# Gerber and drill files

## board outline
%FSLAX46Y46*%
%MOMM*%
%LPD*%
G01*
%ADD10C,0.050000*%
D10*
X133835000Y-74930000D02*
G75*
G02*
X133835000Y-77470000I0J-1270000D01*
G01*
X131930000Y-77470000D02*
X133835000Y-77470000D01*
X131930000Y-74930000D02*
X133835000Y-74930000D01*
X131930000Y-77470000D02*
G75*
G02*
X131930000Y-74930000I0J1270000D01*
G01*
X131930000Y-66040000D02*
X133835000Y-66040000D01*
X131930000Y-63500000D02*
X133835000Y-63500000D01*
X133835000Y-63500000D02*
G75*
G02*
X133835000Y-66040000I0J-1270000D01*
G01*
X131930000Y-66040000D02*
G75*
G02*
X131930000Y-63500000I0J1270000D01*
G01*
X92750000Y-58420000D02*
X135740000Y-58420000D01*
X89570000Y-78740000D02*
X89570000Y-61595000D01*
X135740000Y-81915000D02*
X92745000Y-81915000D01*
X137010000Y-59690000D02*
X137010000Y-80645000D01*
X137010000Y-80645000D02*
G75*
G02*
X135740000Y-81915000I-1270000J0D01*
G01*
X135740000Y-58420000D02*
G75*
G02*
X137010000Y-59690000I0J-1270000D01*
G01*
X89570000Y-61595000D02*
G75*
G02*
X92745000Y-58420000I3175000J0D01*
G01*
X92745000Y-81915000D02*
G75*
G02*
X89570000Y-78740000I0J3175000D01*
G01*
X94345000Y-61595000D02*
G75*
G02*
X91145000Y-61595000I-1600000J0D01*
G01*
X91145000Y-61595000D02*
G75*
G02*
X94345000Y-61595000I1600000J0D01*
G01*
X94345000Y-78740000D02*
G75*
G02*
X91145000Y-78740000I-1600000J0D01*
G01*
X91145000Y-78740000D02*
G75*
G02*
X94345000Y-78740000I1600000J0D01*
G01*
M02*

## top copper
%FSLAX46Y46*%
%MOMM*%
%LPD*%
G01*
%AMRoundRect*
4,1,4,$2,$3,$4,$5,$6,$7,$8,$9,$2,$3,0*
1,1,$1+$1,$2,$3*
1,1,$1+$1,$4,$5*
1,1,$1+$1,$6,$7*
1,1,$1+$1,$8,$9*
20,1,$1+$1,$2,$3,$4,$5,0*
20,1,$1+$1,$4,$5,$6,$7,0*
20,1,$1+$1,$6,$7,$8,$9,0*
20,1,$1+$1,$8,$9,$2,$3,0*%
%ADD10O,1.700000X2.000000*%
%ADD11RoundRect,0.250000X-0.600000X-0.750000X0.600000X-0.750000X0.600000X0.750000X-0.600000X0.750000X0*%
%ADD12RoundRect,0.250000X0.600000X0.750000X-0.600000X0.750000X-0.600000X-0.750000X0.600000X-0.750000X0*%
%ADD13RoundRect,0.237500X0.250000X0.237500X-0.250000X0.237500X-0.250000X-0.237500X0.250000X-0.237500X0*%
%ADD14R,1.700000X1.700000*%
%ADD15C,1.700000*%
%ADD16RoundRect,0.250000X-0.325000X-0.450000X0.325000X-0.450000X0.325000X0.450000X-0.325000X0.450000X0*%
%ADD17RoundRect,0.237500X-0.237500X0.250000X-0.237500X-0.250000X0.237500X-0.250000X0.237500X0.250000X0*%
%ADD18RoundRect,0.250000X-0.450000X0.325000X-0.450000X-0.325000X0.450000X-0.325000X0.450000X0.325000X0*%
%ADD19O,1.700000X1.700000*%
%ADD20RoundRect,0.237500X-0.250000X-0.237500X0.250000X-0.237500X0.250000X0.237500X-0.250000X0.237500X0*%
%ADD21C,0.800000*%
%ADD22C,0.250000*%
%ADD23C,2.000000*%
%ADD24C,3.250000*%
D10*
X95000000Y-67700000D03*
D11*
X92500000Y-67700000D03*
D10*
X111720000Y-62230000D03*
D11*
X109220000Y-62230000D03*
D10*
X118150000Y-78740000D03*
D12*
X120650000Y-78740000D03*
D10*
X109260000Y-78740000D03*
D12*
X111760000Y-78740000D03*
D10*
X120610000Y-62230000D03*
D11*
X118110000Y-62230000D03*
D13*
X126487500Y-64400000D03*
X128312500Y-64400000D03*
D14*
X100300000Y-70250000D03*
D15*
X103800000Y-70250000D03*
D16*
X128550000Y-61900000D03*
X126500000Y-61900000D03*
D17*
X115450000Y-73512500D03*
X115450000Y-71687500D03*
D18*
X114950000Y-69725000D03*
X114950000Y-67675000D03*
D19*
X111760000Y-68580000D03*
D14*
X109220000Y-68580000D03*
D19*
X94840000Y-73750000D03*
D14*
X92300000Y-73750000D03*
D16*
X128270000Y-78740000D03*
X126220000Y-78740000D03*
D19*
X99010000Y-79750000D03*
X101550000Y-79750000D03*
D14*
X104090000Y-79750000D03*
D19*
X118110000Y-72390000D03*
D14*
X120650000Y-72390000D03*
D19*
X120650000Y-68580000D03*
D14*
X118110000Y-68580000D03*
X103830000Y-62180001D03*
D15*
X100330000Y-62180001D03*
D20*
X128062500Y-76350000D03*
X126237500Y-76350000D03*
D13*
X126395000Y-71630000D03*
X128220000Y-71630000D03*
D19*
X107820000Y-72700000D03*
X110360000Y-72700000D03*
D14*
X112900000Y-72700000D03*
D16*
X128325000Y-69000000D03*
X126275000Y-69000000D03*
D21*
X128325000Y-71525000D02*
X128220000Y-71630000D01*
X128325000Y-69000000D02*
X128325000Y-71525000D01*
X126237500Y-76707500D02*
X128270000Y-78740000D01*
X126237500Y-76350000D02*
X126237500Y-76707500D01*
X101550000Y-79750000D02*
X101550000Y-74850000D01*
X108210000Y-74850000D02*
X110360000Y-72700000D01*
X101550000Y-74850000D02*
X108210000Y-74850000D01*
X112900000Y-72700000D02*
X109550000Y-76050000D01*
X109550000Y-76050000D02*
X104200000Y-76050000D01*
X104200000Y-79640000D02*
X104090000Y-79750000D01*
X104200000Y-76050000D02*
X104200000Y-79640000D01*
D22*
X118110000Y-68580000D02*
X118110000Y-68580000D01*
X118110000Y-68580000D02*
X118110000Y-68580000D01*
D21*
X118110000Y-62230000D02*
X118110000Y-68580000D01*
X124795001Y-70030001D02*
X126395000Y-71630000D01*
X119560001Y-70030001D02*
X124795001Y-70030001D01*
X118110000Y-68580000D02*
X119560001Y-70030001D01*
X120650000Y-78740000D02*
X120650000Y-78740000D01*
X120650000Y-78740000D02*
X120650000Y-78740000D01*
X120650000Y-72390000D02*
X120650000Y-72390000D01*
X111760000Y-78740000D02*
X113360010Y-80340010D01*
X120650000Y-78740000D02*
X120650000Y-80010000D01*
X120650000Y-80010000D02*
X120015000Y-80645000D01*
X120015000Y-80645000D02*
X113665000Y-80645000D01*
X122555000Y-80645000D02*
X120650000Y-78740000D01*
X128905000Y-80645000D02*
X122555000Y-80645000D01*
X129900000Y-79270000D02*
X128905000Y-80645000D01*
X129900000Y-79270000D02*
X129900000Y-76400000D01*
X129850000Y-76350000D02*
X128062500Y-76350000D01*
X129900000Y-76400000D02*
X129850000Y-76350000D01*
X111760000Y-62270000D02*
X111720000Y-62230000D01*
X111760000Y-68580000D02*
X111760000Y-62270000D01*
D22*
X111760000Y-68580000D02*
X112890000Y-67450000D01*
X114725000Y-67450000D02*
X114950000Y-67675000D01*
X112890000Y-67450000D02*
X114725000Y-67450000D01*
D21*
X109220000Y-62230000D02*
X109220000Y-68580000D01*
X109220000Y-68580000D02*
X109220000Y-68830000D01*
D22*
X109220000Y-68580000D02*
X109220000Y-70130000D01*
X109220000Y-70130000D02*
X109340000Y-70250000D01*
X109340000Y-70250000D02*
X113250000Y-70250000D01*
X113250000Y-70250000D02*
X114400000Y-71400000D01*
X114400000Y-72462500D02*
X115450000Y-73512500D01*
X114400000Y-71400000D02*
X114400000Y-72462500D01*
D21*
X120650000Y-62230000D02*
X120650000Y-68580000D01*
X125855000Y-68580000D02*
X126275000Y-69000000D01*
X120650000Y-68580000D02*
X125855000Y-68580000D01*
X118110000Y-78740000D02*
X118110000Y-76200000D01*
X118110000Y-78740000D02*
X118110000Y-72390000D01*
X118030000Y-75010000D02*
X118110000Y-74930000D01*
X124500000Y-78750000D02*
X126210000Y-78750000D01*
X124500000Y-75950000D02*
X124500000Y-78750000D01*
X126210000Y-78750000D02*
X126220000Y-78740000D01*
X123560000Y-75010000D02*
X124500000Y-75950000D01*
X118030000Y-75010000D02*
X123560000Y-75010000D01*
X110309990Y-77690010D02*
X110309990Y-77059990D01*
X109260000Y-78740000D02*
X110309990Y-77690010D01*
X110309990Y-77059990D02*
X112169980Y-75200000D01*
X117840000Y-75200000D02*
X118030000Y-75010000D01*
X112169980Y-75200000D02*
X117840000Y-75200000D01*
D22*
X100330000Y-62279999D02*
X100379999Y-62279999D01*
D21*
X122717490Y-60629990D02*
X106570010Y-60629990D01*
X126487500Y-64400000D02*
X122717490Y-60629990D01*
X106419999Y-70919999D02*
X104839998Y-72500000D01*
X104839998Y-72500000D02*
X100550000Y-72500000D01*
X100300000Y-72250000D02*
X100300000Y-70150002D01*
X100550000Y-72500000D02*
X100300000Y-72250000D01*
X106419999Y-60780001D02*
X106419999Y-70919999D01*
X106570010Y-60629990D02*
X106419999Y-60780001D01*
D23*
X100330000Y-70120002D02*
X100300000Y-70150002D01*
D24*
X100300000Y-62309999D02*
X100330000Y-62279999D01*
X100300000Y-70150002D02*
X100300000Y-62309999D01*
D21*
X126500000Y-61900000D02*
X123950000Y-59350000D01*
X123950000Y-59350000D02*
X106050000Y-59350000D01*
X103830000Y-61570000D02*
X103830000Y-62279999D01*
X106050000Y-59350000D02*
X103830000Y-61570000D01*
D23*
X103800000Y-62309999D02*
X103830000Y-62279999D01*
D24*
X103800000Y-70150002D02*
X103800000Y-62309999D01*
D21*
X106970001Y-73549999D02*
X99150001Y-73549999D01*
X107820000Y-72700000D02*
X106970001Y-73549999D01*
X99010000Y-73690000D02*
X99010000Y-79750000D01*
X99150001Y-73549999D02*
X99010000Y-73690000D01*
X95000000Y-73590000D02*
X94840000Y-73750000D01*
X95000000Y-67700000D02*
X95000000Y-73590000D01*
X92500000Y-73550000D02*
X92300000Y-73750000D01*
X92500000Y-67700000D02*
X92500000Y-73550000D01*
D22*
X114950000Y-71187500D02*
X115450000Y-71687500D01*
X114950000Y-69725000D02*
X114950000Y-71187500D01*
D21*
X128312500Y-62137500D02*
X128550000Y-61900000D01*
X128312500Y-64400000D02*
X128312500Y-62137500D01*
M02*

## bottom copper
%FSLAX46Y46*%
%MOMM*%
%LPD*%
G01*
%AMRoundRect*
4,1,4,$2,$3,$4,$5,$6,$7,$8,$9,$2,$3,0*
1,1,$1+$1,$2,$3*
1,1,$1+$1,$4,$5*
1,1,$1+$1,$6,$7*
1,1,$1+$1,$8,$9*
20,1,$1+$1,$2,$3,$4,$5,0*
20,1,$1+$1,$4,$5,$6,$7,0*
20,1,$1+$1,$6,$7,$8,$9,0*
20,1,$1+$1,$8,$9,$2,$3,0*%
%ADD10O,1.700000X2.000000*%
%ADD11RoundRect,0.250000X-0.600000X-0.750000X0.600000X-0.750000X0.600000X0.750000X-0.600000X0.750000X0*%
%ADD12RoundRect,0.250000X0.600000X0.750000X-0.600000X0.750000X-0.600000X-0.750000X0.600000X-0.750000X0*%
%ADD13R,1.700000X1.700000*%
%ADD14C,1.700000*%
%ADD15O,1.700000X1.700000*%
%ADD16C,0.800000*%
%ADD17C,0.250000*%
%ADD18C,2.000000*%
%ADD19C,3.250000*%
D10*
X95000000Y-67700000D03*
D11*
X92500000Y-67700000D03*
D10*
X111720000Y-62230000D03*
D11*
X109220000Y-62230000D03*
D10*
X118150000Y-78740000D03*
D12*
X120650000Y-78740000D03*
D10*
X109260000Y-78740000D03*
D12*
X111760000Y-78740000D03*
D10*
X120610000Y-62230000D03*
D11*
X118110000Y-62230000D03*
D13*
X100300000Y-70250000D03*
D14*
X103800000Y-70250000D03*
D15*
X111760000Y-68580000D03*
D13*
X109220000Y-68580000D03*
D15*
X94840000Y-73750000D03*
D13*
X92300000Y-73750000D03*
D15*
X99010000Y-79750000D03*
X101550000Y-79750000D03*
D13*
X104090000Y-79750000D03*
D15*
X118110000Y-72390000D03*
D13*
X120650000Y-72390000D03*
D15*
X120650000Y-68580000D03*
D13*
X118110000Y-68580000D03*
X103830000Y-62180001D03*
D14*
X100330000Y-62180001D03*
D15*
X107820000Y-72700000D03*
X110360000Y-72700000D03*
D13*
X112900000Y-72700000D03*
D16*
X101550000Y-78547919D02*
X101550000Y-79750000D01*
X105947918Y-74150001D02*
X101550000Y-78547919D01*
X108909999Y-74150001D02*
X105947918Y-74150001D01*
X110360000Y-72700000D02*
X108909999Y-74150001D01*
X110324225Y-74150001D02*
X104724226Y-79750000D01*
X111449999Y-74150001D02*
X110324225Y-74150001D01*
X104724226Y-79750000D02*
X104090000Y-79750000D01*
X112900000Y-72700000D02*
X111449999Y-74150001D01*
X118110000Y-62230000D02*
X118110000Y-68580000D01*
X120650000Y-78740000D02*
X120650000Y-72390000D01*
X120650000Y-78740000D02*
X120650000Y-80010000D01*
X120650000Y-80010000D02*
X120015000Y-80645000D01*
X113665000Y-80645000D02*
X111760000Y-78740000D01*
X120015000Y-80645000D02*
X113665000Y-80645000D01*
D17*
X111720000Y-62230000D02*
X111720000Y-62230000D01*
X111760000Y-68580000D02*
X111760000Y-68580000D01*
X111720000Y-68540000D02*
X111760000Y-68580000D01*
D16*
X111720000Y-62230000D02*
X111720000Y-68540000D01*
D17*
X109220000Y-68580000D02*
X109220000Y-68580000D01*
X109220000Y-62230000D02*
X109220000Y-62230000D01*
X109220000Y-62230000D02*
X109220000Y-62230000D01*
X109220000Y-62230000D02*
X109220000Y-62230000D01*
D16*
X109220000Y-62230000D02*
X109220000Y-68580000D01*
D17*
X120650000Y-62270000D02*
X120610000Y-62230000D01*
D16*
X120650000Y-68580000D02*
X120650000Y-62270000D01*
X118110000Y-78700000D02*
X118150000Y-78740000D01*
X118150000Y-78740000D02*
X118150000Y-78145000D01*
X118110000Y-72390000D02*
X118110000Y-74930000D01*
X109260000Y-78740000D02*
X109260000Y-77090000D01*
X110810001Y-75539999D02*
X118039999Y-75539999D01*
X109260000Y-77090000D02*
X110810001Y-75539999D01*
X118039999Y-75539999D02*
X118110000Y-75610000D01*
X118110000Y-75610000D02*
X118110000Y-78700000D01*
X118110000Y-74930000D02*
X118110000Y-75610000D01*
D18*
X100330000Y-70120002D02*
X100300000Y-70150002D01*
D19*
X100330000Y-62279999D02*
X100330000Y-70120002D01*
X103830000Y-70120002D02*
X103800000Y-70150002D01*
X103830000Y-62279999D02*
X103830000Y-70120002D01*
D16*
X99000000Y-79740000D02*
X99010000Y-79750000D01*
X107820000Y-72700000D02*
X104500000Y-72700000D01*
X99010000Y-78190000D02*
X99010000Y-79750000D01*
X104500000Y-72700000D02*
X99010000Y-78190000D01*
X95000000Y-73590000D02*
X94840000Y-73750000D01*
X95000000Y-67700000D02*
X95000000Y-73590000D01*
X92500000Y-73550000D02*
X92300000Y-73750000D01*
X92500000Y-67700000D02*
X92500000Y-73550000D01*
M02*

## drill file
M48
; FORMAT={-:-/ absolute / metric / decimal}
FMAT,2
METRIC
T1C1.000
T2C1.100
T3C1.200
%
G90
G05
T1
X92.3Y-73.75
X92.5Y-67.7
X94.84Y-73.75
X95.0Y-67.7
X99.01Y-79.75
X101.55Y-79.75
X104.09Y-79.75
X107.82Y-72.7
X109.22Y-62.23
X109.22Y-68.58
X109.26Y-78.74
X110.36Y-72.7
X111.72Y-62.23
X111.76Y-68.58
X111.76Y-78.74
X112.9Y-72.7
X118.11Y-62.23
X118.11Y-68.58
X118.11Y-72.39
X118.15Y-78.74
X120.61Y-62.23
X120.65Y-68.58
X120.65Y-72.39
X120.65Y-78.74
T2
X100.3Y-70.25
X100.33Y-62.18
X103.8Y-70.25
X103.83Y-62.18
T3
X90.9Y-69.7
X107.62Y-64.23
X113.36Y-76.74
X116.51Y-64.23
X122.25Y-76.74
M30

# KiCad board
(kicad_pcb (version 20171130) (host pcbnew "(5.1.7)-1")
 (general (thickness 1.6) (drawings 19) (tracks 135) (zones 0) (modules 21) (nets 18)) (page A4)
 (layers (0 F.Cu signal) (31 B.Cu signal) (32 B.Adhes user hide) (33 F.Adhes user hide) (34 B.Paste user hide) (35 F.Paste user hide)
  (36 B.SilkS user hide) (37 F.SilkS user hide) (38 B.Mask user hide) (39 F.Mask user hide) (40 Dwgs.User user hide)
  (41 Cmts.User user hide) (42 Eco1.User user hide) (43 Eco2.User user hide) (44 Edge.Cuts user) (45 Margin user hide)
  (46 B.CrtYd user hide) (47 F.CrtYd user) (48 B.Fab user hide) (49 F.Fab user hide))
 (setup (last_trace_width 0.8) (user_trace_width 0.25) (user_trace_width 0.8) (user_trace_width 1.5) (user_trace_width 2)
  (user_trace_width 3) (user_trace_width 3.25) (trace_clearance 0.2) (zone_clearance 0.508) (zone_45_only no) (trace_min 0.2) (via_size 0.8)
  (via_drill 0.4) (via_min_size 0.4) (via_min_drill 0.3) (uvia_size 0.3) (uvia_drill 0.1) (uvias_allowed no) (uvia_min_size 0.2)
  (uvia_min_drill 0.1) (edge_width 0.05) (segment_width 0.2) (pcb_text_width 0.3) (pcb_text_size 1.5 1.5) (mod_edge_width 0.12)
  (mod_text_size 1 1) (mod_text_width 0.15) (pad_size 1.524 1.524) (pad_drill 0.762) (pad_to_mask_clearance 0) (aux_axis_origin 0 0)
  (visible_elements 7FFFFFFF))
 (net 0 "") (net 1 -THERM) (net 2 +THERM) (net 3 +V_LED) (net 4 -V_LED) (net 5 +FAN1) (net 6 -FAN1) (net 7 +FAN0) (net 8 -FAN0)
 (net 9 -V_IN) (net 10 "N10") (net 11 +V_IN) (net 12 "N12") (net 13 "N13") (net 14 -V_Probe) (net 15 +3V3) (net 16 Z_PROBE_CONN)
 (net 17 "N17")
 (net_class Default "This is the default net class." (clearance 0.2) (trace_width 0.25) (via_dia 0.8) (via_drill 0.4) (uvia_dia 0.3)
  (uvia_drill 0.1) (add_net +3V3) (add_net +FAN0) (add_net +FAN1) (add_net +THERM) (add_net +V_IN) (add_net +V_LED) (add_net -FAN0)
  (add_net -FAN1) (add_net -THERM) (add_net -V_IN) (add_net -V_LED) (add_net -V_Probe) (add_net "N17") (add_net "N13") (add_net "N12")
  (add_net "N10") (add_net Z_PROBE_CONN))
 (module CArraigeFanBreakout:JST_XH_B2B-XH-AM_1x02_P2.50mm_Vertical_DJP (layer F.Cu) (at 92.5 67.7)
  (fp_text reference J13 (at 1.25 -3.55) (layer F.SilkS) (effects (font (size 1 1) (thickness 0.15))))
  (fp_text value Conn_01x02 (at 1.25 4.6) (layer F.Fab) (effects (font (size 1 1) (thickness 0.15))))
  (pad "" np_thru_hole circle (at -1.6 2) (size 1.2 1.2) (drill 1.2) (layers *.Cu *.Mask))
  (pad 2 thru_hole oval (at 2.5 0) (size 1.7 2) (drill 1) (layers *.Cu *.Mask) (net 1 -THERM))
  (pad 1 thru_hole roundrect (at 0 0) (size 1.7 2) (drill 1) (layers *.Cu *.Mask) (roundrect_rratio 0.147059) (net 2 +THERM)))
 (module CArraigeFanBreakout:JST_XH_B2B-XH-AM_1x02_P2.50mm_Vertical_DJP (layer F.Cu) (at 109.22 62.23)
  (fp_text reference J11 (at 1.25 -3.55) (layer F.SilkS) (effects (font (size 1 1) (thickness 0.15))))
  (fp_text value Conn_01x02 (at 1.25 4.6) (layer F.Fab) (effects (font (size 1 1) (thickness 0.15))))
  (pad "" np_thru_hole circle (at -1.6 2) (size 1.2 1.2) (drill 1.2) (layers *.Cu *.Mask))
  (pad 2 thru_hole oval (at 2.5 0) (size 1.7 2) (drill 1) (layers *.Cu *.Mask) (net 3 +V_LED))
  (pad 1 thru_hole roundrect (at 0 0) (size 1.7 2) (drill 1) (layers *.Cu *.Mask) (roundrect_rratio 0.147059) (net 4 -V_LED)))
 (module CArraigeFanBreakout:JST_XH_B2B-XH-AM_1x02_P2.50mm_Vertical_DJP (layer F.Cu) (at 120.65 78.74 180)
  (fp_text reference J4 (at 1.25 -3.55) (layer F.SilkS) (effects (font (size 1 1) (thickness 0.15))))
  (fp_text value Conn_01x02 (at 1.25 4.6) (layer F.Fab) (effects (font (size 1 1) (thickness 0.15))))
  (pad "" np_thru_hole circle (at -1.6 2 180) (size 1.2 1.2) (drill 1.2) (layers *.Cu *.Mask))
  (pad 2 thru_hole oval (at 2.5 0 180) (size 1.7 2) (drill 1) (layers *.Cu *.Mask) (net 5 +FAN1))
  (pad 1 thru_hole roundrect (at 0 0 180) (size 1.7 2) (drill 1) (layers *.Cu *.Mask) (roundrect_rratio 0.147059) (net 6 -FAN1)))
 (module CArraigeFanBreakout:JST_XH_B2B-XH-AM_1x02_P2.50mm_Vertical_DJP (layer F.Cu) (at 111.76 78.74 180)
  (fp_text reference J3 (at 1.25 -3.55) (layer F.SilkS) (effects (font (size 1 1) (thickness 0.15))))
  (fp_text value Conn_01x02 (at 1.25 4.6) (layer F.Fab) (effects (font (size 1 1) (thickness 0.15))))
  (pad "" np_thru_hole circle (at -1.6 2 180) (size 1.2 1.2) (drill 1.2) (layers *.Cu *.Mask))
  (pad 2 thru_hole oval (at 2.5 0 180) (size 1.7 2) (drill 1) (layers *.Cu *.Mask) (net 5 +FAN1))
  (pad 1 thru_hole roundrect (at 0 0 180) (size 1.7 2) (drill 1) (layers *.Cu *.Mask) (roundrect_rratio 0.147059) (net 6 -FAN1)))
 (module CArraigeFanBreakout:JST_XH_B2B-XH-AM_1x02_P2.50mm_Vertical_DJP (layer F.Cu) (at 118.11 62.23)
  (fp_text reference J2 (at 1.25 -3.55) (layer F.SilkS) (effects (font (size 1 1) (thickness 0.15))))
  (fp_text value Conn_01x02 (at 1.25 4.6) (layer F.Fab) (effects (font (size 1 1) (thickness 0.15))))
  (pad "" np_thru_hole circle (at -1.6 2) (size 1.2 1.2) (drill 1.2) (layers *.Cu *.Mask))
  (pad 2 thru_hole oval (at 2.5 0) (size 1.7 2) (drill 1) (layers *.Cu *.Mask) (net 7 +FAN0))
  (pad 1 thru_hole roundrect (at 0 0) (size 1.7 2) (drill 1) (layers *.Cu *.Mask) (roundrect_rratio 0.147059) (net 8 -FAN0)))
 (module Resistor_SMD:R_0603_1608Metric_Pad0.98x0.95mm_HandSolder (layer F.Cu) (at 127.4 64.4 180)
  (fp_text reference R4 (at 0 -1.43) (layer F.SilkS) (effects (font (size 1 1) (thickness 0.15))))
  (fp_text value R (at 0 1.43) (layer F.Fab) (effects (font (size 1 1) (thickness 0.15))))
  (pad 2 smd roundrect (at 0.9125 0 180) (size 0.975 0.95) (layers F.Cu F.Paste F.Mask) (roundrect_rratio 0.25) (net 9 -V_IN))
  (pad 1 smd roundrect (at -0.9125 0 180) (size 0.975 0.95) (layers F.Cu F.Paste F.Mask) (roundrect_rratio 0.25) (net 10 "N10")))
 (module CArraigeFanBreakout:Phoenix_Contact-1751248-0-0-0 (layer F.Cu) (at 102.05 70.200001)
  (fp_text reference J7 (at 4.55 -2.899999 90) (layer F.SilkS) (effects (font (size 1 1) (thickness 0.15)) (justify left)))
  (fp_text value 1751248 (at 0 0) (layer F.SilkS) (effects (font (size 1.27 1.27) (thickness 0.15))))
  (pad 1 thru_hole rect (at -1.75 0.049999) (size 1.7 1.7) (drill 1.1) (layers *.Cu) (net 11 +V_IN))
  (pad 2 thru_hole circle (at 1.75 0.049999) (size 1.7 1.7) (drill 1.1) (layers *.Cu) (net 9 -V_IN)))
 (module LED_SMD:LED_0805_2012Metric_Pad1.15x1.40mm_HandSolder (layer F.Cu) (at 127.525 61.9)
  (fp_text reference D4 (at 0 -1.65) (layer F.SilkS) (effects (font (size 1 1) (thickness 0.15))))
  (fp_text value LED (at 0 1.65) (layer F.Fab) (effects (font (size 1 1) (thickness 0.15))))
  (pad 2 smd roundrect (at 1.025 0) (size 1.15 1.4) (layers F.Cu F.Paste F.Mask) (roundrect_rratio 0.217391) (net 10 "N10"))
  (pad 1 smd roundrect (at -1.025 0) (size 1.15 1.4) (layers F.Cu F.Paste F.Mask) (roundrect_rratio 0.217391) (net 11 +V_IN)))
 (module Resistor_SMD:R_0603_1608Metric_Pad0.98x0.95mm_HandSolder (layer F.Cu) (at 115.45 72.6 270)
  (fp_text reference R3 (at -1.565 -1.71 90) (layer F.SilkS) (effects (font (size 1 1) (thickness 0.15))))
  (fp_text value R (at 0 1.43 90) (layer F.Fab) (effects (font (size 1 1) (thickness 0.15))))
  (pad 2 smd roundrect (at 0.9125 0 270) (size 0.975 0.95) (layers F.Cu F.Paste F.Mask) (roundrect_rratio 0.25) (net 4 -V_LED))
  (pad 1 smd roundrect (at -0.9125 0 270) (size 0.975 0.95) (layers F.Cu F.Paste F.Mask) (roundrect_rratio 0.25) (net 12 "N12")))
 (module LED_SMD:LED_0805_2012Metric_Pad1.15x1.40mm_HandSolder (layer F.Cu) (at 114.95 68.7 270)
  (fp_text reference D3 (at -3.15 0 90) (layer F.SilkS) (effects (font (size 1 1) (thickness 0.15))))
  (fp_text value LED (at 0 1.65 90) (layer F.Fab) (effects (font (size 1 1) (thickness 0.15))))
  (pad 2 smd roundrect (at 1.025 0 270) (size 1.15 1.4) (layers F.Cu F.Paste F.Mask) (roundrect_rratio 0.217391) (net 12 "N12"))
  (pad 1 smd roundrect (at -1.025 0 270) (size 1.15 1.4) (layers F.Cu F.Paste F.Mask) (roundrect_rratio 0.217391) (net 3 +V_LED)))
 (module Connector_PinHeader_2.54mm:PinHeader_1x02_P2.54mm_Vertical (layer F.Cu) (at 109.22 68.58 90)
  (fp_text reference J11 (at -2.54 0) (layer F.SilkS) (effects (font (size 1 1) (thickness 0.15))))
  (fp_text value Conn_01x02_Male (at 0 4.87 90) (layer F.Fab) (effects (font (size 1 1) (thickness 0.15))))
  (pad 2 thru_hole oval (at 0 2.54 90) (size 1.7 1.7) (drill 1) (layers *.Cu *.Mask) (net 3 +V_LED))
  (pad 1 thru_hole rect (at 0 0 90) (size 1.7 1.7) (drill 1) (layers *.Cu *.Mask) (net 4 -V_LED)))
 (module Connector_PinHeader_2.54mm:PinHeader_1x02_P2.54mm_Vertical (layer F.Cu) (at 92.3 73.75 90)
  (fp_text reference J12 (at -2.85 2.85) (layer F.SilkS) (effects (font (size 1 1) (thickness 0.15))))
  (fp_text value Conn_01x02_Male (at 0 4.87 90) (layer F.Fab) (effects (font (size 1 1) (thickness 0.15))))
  (pad 2 thru_hole oval (at 0 2.54 90) (size 1.7 1.7) (drill 1) (layers *.Cu *.Mask) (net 1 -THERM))
  (pad 1 thru_hole rect (at 0 0 90) (size 1.7 1.7) (drill 1) (layers *.Cu *.Mask) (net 2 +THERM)))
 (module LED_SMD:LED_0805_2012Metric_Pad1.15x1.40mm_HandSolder (layer F.Cu) (at 127.245 78.74)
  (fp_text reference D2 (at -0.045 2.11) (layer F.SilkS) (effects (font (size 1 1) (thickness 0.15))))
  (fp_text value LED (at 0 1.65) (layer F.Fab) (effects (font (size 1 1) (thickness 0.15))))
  (pad 2 smd roundrect (at 1.025 0) (size 1.15 1.4) (layers F.Cu F.Paste F.Mask) (roundrect_rratio 0.217391) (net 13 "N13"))
  (pad 1 smd roundrect (at -1.025 0) (size 1.15 1.4) (layers F.Cu F.Paste F.Mask) (roundrect_rratio 0.217391) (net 5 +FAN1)))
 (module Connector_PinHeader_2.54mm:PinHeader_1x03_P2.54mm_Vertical (layer F.Cu) (at 104.09 79.75 270)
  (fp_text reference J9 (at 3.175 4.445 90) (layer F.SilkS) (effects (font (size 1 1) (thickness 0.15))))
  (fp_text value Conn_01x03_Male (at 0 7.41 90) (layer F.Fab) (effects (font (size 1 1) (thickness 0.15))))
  (pad 3 thru_hole oval (at 0 5.08 270) (size 1.7 1.7) (drill 1) (layers *.Cu *.Mask) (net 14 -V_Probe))
  (pad 2 thru_hole oval (at 0 2.54 270) (size 1.7 1.7) (drill 1) (layers *.Cu *.Mask) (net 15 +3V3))
  (pad 1 thru_hole rect (at 0 0 270) (size 1.7 1.7) (drill 1) (layers *.Cu *.Mask) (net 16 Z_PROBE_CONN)))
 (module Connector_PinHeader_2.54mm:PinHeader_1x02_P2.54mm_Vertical (layer F.Cu) (at 120.65 72.39 270)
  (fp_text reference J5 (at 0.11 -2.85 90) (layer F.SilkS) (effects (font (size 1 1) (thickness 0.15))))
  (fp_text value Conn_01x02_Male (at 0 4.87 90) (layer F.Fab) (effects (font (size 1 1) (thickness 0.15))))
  (pad 2 thru_hole oval (at 0 2.54 270) (size 1.7 1.7) (drill 1) (layers *.Cu *.Mask) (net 5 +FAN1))
  (pad 1 thru_hole rect (at 0 0 270) (size 1.7 1.7) (drill 1) (layers *.Cu *.Mask) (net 6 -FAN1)))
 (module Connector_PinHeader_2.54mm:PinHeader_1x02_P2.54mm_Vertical (layer F.Cu) (at 118.11 68.58 90)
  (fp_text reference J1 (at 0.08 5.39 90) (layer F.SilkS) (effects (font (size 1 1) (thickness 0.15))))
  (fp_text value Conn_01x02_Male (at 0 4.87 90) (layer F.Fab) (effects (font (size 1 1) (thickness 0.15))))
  (pad 2 thru_hole oval (at 0 2.54 90) (size 1.7 1.7) (drill 1) (layers *.Cu *.Mask) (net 7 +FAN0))
  (pad 1 thru_hole rect (at 0 0 90) (size 1.7 1.7) (drill 1) (layers *.Cu *.Mask) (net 8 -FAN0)))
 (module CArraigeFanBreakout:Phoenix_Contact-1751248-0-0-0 (layer F.Cu) (at 102.08 62.23 180)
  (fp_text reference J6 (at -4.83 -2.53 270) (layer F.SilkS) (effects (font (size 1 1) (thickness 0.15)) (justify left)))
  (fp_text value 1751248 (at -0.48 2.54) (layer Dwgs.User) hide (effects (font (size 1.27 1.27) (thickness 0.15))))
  (pad 1 thru_hole rect (at -1.75 0.049999 180) (size 1.7 1.7) (drill 1.1) (layers *.Cu) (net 9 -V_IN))
  (pad 2 thru_hole circle (at 1.75 0.049999 180) (size 1.7 1.7) (drill 1.1) (layers *.Cu) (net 11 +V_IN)))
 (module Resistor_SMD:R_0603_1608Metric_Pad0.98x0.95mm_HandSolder (layer F.Cu) (at 127.15 76.35)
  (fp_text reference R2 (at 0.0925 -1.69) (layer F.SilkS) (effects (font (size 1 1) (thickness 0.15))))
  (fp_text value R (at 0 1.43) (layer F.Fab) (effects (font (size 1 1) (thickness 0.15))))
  (pad 2 smd roundrect (at 0.9125 0) (size 0.975 0.95) (layers F.Cu F.Paste F.Mask) (roundrect_rratio 0.25) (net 6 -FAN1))
  (pad 1 smd roundrect (at -0.9125 0) (size 0.975 0.95) (layers F.Cu F.Paste F.Mask) (roundrect_rratio 0.25) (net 13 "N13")))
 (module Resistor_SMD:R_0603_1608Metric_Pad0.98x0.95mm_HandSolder (layer F.Cu) (at 127.3075 71.63 180)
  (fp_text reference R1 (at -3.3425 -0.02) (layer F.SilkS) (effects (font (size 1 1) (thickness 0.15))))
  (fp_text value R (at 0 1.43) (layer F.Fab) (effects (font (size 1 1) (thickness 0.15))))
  (pad 2 smd roundrect (at 0.9125 0 180) (size 0.975 0.95) (layers F.Cu F.Paste F.Mask) (roundrect_rratio 0.25) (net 8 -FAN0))
  (pad 1 smd roundrect (at -0.9125 0 180) (size 0.975 0.95) (layers F.Cu F.Paste F.Mask) (roundrect_rratio 0.25) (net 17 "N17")))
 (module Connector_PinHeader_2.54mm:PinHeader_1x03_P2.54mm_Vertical (layer F.Cu) (at 112.9 72.7 270)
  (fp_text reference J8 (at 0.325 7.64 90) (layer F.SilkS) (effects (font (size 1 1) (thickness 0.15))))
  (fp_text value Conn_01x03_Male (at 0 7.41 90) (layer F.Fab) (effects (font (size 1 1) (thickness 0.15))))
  (pad 3 thru_hole oval (at 0 5.08 270) (size 1.7 1.7) (drill 1) (layers *.Cu *.Mask) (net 14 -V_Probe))
  (pad 2 thru_hole oval (at 0 2.54 270) (size 1.7 1.7) (drill 1) (layers *.Cu *.Mask) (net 15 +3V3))
  (pad 1 thru_hole rect (at 0 0 270) (size 1.7 1.7) (drill 1) (layers *.Cu *.Mask) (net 16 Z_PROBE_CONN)))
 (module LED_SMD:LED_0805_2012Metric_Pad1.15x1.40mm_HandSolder (layer F.Cu) (at 127.3 69)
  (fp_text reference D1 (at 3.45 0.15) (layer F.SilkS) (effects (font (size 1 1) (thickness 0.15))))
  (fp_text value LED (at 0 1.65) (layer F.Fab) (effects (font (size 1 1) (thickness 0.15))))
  (pad 2 smd roundrect (at 1.025 0) (size 1.15 1.4) (layers F.Cu F.Paste F.Mask) (roundrect_rratio 0.217391) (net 17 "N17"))
  (pad 1 smd roundrect (at -1.025 0) (size 1.15 1.4) (layers F.Cu F.Paste F.Mask) (roundrect_rratio 0.217391) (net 7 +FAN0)))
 (gr_arc (start 133.835 76.2) (end 133.835 77.47) (angle -180) (layer Edge.Cuts) (width 0.05))
 (gr_line (start 131.93 77.47) (end 133.835 77.47) (layer Edge.Cuts) (width 0.05))
 (gr_line (start 131.93 74.93) (end 133.835 74.93) (layer Edge.Cuts) (width 0.05))
 (gr_arc (start 131.93 76.2) (end 131.93 74.93) (angle -180) (layer Edge.Cuts) (width 0.05))
 (gr_line (start 131.93 66.04) (end 133.835 66.04) (layer Edge.Cuts) (width 0.05))
 (gr_line (start 131.93 63.5) (end 133.835 63.5) (layer Edge.Cuts) (width 0.05))
 (gr_arc (start 133.835 64.77) (end 133.835 66.04) (angle -180) (layer Edge.Cuts) (width 0.05))
 (gr_arc (start 131.93 64.77) (end 131.93 63.5) (angle -180) (layer Edge.Cuts) (width 0.05))
 (gr_line (start 92.75 58.42) (end 135.74 58.42) (layer Edge.Cuts) (width 0.05))
 (gr_line (start 89.57 78.74) (end 89.57 61.595) (layer Edge.Cuts) (width 0.05))
 (gr_line (start 135.74 81.915) (end 92.745 81.915) (layer Edge.Cuts) (width 0.05))
 (gr_line (start 137.01 59.69) (end 137.01 80.645) (layer Edge.Cuts) (width 0.05))
 (gr_arc (start 135.74 80.645) (end 135.74 81.915) (angle -90) (layer Edge.Cuts) (width 0.05))
 (gr_arc (start 135.74 59.69) (end 137.01 59.69) (angle -90) (layer Edge.Cuts) (width 0.05))
 (gr_arc (start 92.745 61.595) (end 92.745 58.42) (angle -90) (layer Edge.Cuts) (width 0.05))
 (gr_arc (start 92.745 78.74) (end 89.57 78.74) (angle -90) (layer Edge.Cuts) (width 0.05))
 (gr_circle (center 92.745 61.595) (end 92.745 63.195) (layer Edge.Cuts) (width 0.05))
 (gr_circle (center 92.745 78.74) (end 92.745 80.34) (layer Edge.Cuts) (width 0.05))
 (segment (start 128.325 71.525) (end 128.22 71.63) (width 0.8) (layer F.Cu) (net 17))
 (segment (start 128.325 69) (end 128.325 71.525) (width 0.8) (layer F.Cu) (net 17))
 (segment (start 126.2375 76.7075) (end 128.27 78.74) (width 0.8) (layer F.Cu) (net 13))
 (segment (start 126.2375 76.35) (end 126.2375 76.7075) (width 0.8) (layer F.Cu) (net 13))
 (segment (start 101.55 79.75) (end 101.55 74.85) (width 0.8) (layer F.Cu) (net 15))
 (segment (start 108.21 74.85) (end 110.36 72.7) (width 0.8) (layer F.Cu) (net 15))
 (segment (start 101.55 74.85) (end 108.21 74.85) (width 0.8) (layer F.Cu) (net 15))
 (segment (start 101.55 78.547919) (end 101.55 79.75) (width 0.8) (layer B.Cu) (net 15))
 (segment (start 105.947918 74.150001) (end 101.55 78.547919) (width 0.8) (layer B.Cu) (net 15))
 (segment (start 108.909999 74.150001) (end 105.947918 74.150001) (width 0.8) (layer B.Cu) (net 15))
 (segment (start 110.36 72.7) (end 108.909999 74.150001) (width 0.8) (layer B.Cu) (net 15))
 (segment (start 112.9 72.7) (end 109.55 76.05) (width 0.8) (layer F.Cu) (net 16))
 (segment (start 109.55 76.05) (end 104.2 76.05) (width 0.8) (layer F.Cu) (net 16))
 (segment (start 104.2 79.64) (end 104.09 79.75) (width 0.8) (layer F.Cu) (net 16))
 (segment (start 104.2 76.05) (end 104.2 79.64) (width 0.8) (layer F.Cu) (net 16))
 (segment (start 110.324225 74.150001) (end 104.724226 79.75) (width 0.8) (layer B.Cu) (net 16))
 (segment (start 111.449999 74.150001) (end 110.324225 74.150001) (width 0.8) (layer B.Cu) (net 16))
 (segment (start 104.724226 79.75) (end 104.09 79.75) (width 0.8) (layer B.Cu) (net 16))
 (segment (start 112.9 72.7) (end 111.449999 74.150001) (width 0.8) (layer B.Cu) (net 16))
 (segment (start 118.11 68.58) (end 118.11 68.58) (width 0.25) (layer F.Cu) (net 8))
 (segment (start 118.11 68.58) (end 118.11 68.58) (width 0.25) (layer F.Cu) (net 8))
 (segment (start 118.11 62.23) (end 118.11 68.58) (width 0.8) (layer F.Cu) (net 8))
 (segment (start 118.11 62.23) (end 118.11 68.58) (width 0.8) (layer B.Cu) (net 8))
 (segment (start 124.795001 70.030001) (end 126.395 71.63) (width 0.8) (layer F.Cu) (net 8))
 (segment (start 119.560001 70.030001) (end 124.795001 70.030001) (width 0.8) (layer F.Cu) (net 8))
 (segment (start 118.11 68.58) (end 119.560001 70.030001) (width 0.8) (layer F.Cu) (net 8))
 (segment (start 120.65 78.74) (end 120.65 78.74) (width 0.8) (layer F.Cu) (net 6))
 (segment (start 120.65 78.74) (end 120.65 78.74) (width 0.8) (layer F.Cu) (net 6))
 (segment (start 120.65 72.39) (end 120.65 72.39) (width 0.8) (layer F.Cu) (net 6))
 (segment (start 120.65 78.74) (end 120.65 72.39) (width 0.8) (layer B.Cu) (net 6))
 (segment (start 120.65 78.74) (end 120.65 80.01) (width 0.8) (layer B.Cu) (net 6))
 (segment (start 120.65 80.01) (end 120.015 80.645) (width 0.8) (layer B.Cu) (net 6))
 (segment (start 113.665 80.645) (end 111.76 78.74) (width 0.8) (layer B.Cu) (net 6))
 (segment (start 120.015 80.645) (end 113.665 80.645) (width 0.8) (layer B.Cu) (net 6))
 (segment (start 111.76 78.74) (end 113.36001 80.34001) (width 0.8) (layer F.Cu) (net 6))
 (segment (start 120.65 78.74) (end 120.65 80.01) (width 0.8) (layer F.Cu) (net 6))
 (segment (start 120.65 80.01) (end 120.015 80.645) (width 0.8) (layer F.Cu) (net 6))
 (segment (start 120.015 80.645) (end 113.665 80.645) (width 0.8) (layer F.Cu) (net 6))
 (segment (start 122.555 80.645) (end 120.65 78.74) (width 0.8) (layer F.Cu) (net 6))
 (segment (start 128.905 80.645) (end 122.555 80.645) (width 0.8) (layer F.Cu) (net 6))
 (segment (start 129.9 79.27) (end 128.905 80.645) (width 0.8) (layer F.Cu) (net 6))
 (segment (start 129.9 79.27) (end 129.9 76.4) (width 0.8) (layer F.Cu) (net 6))
 (segment (start 129.85 76.35) (end 128.0625 76.35) (width 0.8) (layer F.Cu) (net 6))
 (segment (start 129.9 76.4) (end 129.85 76.35) (width 0.8) (layer F.Cu) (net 6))
 (segment (start 111.72 62.23) (end 111.72 62.23) (width 0.25) (layer B.Cu) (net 3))
 (segment (start 111.76 68.58) (end 111.76 68.58) (width 0.25) (layer B.Cu) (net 3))
 (segment (start 111.72 68.54) (end 111.76 68.58) (width 0.25) (layer B.Cu) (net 3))
 (segment (start 111.72 62.23) (end 111.72 68.54) (width 0.8) (layer B.Cu) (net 3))
 (segment (start 111.76 62.27) (end 111.72 62.23) (width 0.8) (layer F.Cu) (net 3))
 (segment (start 111.76 68.58) (end 111.76 62.27) (width 0.8) (layer F.Cu) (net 3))
 (segment (start 111.76 68.58) (end 112.89 67.45) (width 0.25) (layer F.Cu) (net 3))
 (segment (start 114.725 67.45) (end 114.95 67.675) (width 0.25) (layer F.Cu) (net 3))
 (segment (start 112.89 67.45) (end 114.725 67.45) (width 0.25) (layer F.Cu) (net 3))
 (segment (start 109.22 68.58) (end 109.22 68.58) (width 0.25) (layer B.Cu) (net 4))
 (segment (start 109.22 62.23) (end 109.22 62.23) (width 0.25) (layer B.Cu) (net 4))
 (segment (start 109.22 62.23) (end 109.22 62.23) (width 0.25) (layer B.Cu) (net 4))
 (segment (start 109.22 62.23) (end 109.22 62.23) (width 0.25) (layer B.Cu) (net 4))
 (segment (start 109.22 62.23) (end 109.22 68.58) (width 0.8) (layer B.Cu) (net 4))
 (segment (start 109.22 62.23) (end 109.22 68.58) (width 0.8) (layer F.Cu) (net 4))
 (segment (start 109.22 68.58) (end 109.22 68.83) (width 0.8) (layer F.Cu) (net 4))
 (segment (start 109.22 68.58) (end 109.22 70.13) (width 0.25) (layer F.Cu) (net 4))
 (segment (start 109.22 70.13) (end 109.34 70.25) (width 0.25) (layer F.Cu) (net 4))
 (segment (start 109.34 70.25) (end 113.25 70.25) (width 0.25) (layer F.Cu) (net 4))
 (segment (start 113.25 70.25) (end 114.4 71.4) (width 0.25) (layer F.Cu) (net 4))
 (segment (start 114.4 72.4625) (end 115.45 73.5125) (width 0.25) (layer F.Cu) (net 4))
 (segment (start 114.4 71.4) (end 114.4 72.4625) (width 0.25) (layer F.Cu) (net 4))
 (segment (start 120.65 62.27) (end 120.61 62.23) (width 0.25) (layer B.Cu) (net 7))
 (segment (start 120.65 68.58) (end 120.65 62.27) (width 0.8) (layer B.Cu) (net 7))
 (segment (start 120.65 62.23) (end 120.65 68.58) (width 0.8) (layer F.Cu) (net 7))
 (segment (start 125.855 68.58) (end 126.275 69) (width 0.8) (layer F.Cu) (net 7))
 (segment (start 120.65 68.58) (end 125.855 68.58) (width 0.8) (layer F.Cu) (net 7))
 (segment (start 118.11 78.7) (end 118.15 78.74) (width 0.8) (layer B.Cu) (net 5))
 (segment (start 118.15 78.74) (end 118.15 78.145) (width 0.8) (layer B.Cu) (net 5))
 (segment (start 118.11 78.74) (end 118.11 76.2) (width 0.8) (layer F.Cu) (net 5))
 (segment (start 118.11 78.74) (end 118.11 72.39) (width 0.8) (layer F.Cu) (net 5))
 (segment (start 118.11 72.39) (end 118.11 74.93) (width 0.8) (layer B.Cu) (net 5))
 (segment (start 118.03 75.01) (end 118.11 74.93) (width 0.8) (layer F.Cu) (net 5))
 (segment (start 124.5 78.75) (end 126.21 78.75) (width 0.8) (layer F.Cu) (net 5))
 (segment (start 124.5 75.95) (end 124.5 78.75) (width 0.8) (layer F.Cu) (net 5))
 (segment (start 126.21 78.75) (end 126.22 78.74) (width 0.8) (layer F.Cu) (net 5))
 (segment (start 123.56 75.01) (end 124.5 75.95) (width 0.8) (layer F.Cu) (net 5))
 (segment (start 118.03 75.01) (end 123.56 75.01) (width 0.8) (layer F.Cu) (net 5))
 (segment (start 110.30999 77.69001) (end 110.30999 77.05999) (width 0.8) (layer F.Cu) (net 5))
 (segment (start 109.26 78.74) (end 110.30999 77.69001) (width 0.8) (layer F.Cu) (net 5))
 (segment (start 110.30999 77.05999) (end 112.16998 75.2) (width 0.8) (layer F.Cu) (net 5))
 (segment (start 117.84 75.2) (end 118.03 75.01) (width 0.8) (layer F.Cu) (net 5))
 (segment (start 112.16998 75.2) (end 117.84 75.2) (width 0.8) (layer F.Cu) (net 5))
 (segment (start 109.26 78.74) (end 109.26 77.09) (width 0.8) (layer B.Cu) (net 5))
 (segment (start 110.810001 75.539999) (end 118.039999 75.539999) (width 0.8) (layer B.Cu) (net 5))
 (segment (start 109.26 77.09) (end 110.810001 75.539999) (width 0.8) (layer B.Cu) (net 5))
 (segment (start 118.039999 75.539999) (end 118.11 75.61) (width 0.8) (layer B.Cu) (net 5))
 (segment (start 118.11 75.61) (end 118.11 78.7) (width 0.8) (layer B.Cu) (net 5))
 (segment (start 118.11 74.93) (end 118.11 75.61) (width 0.8) (layer B.Cu) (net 5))
 (segment (start 100.33 62.279999) (end 100.379999 62.279999) (width 0.25) (layer F.Cu) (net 9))
 (segment (start 122.71749 60.62999) (end 106.57001 60.62999) (width 0.8) (layer F.Cu) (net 9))
 (segment (start 126.4875 64.4) (end 122.71749 60.62999) (width 0.8) (layer F.Cu) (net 9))
 (segment (start 106.419999 70.919999) (end 104.839998 72.5) (width 0.8) (layer F.Cu) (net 9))
 (segment (start 104.839998 72.5) (end 100.55 72.5) (width 0.8) (layer F.Cu) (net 9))
 (segment (start 100.3 72.25) (end 100.3 70.150002) (width 0.8) (layer F.Cu) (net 9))
 (segment (start 100.55 72.5) (end 100.3 72.25) (width 0.8) (layer F.Cu) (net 9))
 (segment (start 106.419999 60.780001) (end 106.419999 70.919999) (width 0.8) (layer F.Cu) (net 9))
 (segment (start 106.57001 60.62999) (end 106.419999 60.780001) (width 0.8) (layer F.Cu) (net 9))
 (segment (start 100.33 70.120002) (end 100.3 70.150002) (width 2) (layer B.Cu) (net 9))
 (segment (start 100.33 70.120002) (end 100.3 70.150002) (width 2) (layer F.Cu) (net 9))
 (segment (start 100.33 62.279999) (end 100.33 70.120002) (width 3.25) (layer B.Cu) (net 9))
 (segment (start 100.3 62.309999) (end 100.33 62.279999) (width 3.25) (layer F.Cu) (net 9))
 (segment (start 100.3 70.150002) (end 100.3 62.309999) (width 3.25) (layer F.Cu) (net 9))
 (segment (start 126.5 61.9) (end 123.95 59.35) (width 0.8) (layer F.Cu) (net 11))
 (segment (start 123.95 59.35) (end 106.05 59.35) (width 0.8) (layer F.Cu) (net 11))
 (segment (start 103.83 61.57) (end 103.83 62.279999) (width 0.8) (layer F.Cu) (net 11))
 (segment (start 106.05 59.35) (end 103.83 61.57) (width 0.8) (layer F.Cu) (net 11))
 (segment (start 103.8 62.309999) (end 103.83 62.279999) (width 2) (layer F.Cu) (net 11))
 (segment (start 103.83 70.120002) (end 103.8 70.150002) (width 3.25) (layer B.Cu) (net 11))
 (segment (start 103.83 62.279999) (end 103.83 70.120002) (width 3.25) (layer B.Cu) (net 11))
 (segment (start 103.8 70.150002) (end 103.8 62.309999) (width 3.25) (layer F.Cu) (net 11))
 (segment (start 106.970001 73.549999) (end 99.150001 73.549999) (width 0.8) (layer F.Cu) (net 14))
 (segment (start 107.82 72.7) (end 106.970001 73.549999) (width 0.8) (layer F.Cu) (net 14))
 (segment (start 99.01 73.69) (end 99.01 79.75) (width 0.8) (layer F.Cu) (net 14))
 (segment (start 99.150001 73.549999) (end 99.01 73.69) (width 0.8) (layer F.Cu) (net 14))
 (segment (start 99 79.74) (end 99.01 79.75) (width 0.8) (layer B.Cu) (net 14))
 (segment (start 107.82 72.7) (end 104.5 72.7) (width 0.8) (layer B.Cu) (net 14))
 (segment (start 99.01 78.19) (end 99.01 79.75) (width 0.8) (layer B.Cu) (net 14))
 (segment (start 104.5 72.7) (end 99.01 78.19) (width 0.8) (layer B.Cu) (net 14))
 (segment (start 95 73.59) (end 94.84 73.75) (width 0.8) (layer F.Cu) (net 1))
 (segment (start 95 67.7) (end 95 73.59) (width 0.8) (layer F.Cu) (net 1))
 (segment (start 95 73.59) (end 94.84 73.75) (width 0.8) (layer B.Cu) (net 1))
 (segment (start 95 67.7) (end 95 73.59) (width 0.8) (layer B.Cu) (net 1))
 (segment (start 92.5 73.55) (end 92.3 73.75) (width 0.8) (layer F.Cu) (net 2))
 (segment (start 92.5 67.7) (end 92.5 73.55) (width 0.8) (layer F.Cu) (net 2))
 (segment (start 92.5 73.55) (end 92.3 73.75) (width 0.8) (layer B.Cu) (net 2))
 (segment (start 92.5 67.7) (end 92.5 73.55) (width 0.8) (layer B.Cu) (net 2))
 (segment (start 114.95 71.1875) (end 115.45 71.6875) (width 0.25) (layer F.Cu) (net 12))
 (segment (start 114.95 69.725) (end 114.95 71.1875) (width 0.25) (layer F.Cu) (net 12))
 (segment (start 128.3125 62.1375) (end 128.55 61.9) (width 0.8) (layer F.Cu) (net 10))
 (segment (start 128.3125 64.4) (end 128.3125 62.1375) (width 0.8) (layer F.Cu) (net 10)))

